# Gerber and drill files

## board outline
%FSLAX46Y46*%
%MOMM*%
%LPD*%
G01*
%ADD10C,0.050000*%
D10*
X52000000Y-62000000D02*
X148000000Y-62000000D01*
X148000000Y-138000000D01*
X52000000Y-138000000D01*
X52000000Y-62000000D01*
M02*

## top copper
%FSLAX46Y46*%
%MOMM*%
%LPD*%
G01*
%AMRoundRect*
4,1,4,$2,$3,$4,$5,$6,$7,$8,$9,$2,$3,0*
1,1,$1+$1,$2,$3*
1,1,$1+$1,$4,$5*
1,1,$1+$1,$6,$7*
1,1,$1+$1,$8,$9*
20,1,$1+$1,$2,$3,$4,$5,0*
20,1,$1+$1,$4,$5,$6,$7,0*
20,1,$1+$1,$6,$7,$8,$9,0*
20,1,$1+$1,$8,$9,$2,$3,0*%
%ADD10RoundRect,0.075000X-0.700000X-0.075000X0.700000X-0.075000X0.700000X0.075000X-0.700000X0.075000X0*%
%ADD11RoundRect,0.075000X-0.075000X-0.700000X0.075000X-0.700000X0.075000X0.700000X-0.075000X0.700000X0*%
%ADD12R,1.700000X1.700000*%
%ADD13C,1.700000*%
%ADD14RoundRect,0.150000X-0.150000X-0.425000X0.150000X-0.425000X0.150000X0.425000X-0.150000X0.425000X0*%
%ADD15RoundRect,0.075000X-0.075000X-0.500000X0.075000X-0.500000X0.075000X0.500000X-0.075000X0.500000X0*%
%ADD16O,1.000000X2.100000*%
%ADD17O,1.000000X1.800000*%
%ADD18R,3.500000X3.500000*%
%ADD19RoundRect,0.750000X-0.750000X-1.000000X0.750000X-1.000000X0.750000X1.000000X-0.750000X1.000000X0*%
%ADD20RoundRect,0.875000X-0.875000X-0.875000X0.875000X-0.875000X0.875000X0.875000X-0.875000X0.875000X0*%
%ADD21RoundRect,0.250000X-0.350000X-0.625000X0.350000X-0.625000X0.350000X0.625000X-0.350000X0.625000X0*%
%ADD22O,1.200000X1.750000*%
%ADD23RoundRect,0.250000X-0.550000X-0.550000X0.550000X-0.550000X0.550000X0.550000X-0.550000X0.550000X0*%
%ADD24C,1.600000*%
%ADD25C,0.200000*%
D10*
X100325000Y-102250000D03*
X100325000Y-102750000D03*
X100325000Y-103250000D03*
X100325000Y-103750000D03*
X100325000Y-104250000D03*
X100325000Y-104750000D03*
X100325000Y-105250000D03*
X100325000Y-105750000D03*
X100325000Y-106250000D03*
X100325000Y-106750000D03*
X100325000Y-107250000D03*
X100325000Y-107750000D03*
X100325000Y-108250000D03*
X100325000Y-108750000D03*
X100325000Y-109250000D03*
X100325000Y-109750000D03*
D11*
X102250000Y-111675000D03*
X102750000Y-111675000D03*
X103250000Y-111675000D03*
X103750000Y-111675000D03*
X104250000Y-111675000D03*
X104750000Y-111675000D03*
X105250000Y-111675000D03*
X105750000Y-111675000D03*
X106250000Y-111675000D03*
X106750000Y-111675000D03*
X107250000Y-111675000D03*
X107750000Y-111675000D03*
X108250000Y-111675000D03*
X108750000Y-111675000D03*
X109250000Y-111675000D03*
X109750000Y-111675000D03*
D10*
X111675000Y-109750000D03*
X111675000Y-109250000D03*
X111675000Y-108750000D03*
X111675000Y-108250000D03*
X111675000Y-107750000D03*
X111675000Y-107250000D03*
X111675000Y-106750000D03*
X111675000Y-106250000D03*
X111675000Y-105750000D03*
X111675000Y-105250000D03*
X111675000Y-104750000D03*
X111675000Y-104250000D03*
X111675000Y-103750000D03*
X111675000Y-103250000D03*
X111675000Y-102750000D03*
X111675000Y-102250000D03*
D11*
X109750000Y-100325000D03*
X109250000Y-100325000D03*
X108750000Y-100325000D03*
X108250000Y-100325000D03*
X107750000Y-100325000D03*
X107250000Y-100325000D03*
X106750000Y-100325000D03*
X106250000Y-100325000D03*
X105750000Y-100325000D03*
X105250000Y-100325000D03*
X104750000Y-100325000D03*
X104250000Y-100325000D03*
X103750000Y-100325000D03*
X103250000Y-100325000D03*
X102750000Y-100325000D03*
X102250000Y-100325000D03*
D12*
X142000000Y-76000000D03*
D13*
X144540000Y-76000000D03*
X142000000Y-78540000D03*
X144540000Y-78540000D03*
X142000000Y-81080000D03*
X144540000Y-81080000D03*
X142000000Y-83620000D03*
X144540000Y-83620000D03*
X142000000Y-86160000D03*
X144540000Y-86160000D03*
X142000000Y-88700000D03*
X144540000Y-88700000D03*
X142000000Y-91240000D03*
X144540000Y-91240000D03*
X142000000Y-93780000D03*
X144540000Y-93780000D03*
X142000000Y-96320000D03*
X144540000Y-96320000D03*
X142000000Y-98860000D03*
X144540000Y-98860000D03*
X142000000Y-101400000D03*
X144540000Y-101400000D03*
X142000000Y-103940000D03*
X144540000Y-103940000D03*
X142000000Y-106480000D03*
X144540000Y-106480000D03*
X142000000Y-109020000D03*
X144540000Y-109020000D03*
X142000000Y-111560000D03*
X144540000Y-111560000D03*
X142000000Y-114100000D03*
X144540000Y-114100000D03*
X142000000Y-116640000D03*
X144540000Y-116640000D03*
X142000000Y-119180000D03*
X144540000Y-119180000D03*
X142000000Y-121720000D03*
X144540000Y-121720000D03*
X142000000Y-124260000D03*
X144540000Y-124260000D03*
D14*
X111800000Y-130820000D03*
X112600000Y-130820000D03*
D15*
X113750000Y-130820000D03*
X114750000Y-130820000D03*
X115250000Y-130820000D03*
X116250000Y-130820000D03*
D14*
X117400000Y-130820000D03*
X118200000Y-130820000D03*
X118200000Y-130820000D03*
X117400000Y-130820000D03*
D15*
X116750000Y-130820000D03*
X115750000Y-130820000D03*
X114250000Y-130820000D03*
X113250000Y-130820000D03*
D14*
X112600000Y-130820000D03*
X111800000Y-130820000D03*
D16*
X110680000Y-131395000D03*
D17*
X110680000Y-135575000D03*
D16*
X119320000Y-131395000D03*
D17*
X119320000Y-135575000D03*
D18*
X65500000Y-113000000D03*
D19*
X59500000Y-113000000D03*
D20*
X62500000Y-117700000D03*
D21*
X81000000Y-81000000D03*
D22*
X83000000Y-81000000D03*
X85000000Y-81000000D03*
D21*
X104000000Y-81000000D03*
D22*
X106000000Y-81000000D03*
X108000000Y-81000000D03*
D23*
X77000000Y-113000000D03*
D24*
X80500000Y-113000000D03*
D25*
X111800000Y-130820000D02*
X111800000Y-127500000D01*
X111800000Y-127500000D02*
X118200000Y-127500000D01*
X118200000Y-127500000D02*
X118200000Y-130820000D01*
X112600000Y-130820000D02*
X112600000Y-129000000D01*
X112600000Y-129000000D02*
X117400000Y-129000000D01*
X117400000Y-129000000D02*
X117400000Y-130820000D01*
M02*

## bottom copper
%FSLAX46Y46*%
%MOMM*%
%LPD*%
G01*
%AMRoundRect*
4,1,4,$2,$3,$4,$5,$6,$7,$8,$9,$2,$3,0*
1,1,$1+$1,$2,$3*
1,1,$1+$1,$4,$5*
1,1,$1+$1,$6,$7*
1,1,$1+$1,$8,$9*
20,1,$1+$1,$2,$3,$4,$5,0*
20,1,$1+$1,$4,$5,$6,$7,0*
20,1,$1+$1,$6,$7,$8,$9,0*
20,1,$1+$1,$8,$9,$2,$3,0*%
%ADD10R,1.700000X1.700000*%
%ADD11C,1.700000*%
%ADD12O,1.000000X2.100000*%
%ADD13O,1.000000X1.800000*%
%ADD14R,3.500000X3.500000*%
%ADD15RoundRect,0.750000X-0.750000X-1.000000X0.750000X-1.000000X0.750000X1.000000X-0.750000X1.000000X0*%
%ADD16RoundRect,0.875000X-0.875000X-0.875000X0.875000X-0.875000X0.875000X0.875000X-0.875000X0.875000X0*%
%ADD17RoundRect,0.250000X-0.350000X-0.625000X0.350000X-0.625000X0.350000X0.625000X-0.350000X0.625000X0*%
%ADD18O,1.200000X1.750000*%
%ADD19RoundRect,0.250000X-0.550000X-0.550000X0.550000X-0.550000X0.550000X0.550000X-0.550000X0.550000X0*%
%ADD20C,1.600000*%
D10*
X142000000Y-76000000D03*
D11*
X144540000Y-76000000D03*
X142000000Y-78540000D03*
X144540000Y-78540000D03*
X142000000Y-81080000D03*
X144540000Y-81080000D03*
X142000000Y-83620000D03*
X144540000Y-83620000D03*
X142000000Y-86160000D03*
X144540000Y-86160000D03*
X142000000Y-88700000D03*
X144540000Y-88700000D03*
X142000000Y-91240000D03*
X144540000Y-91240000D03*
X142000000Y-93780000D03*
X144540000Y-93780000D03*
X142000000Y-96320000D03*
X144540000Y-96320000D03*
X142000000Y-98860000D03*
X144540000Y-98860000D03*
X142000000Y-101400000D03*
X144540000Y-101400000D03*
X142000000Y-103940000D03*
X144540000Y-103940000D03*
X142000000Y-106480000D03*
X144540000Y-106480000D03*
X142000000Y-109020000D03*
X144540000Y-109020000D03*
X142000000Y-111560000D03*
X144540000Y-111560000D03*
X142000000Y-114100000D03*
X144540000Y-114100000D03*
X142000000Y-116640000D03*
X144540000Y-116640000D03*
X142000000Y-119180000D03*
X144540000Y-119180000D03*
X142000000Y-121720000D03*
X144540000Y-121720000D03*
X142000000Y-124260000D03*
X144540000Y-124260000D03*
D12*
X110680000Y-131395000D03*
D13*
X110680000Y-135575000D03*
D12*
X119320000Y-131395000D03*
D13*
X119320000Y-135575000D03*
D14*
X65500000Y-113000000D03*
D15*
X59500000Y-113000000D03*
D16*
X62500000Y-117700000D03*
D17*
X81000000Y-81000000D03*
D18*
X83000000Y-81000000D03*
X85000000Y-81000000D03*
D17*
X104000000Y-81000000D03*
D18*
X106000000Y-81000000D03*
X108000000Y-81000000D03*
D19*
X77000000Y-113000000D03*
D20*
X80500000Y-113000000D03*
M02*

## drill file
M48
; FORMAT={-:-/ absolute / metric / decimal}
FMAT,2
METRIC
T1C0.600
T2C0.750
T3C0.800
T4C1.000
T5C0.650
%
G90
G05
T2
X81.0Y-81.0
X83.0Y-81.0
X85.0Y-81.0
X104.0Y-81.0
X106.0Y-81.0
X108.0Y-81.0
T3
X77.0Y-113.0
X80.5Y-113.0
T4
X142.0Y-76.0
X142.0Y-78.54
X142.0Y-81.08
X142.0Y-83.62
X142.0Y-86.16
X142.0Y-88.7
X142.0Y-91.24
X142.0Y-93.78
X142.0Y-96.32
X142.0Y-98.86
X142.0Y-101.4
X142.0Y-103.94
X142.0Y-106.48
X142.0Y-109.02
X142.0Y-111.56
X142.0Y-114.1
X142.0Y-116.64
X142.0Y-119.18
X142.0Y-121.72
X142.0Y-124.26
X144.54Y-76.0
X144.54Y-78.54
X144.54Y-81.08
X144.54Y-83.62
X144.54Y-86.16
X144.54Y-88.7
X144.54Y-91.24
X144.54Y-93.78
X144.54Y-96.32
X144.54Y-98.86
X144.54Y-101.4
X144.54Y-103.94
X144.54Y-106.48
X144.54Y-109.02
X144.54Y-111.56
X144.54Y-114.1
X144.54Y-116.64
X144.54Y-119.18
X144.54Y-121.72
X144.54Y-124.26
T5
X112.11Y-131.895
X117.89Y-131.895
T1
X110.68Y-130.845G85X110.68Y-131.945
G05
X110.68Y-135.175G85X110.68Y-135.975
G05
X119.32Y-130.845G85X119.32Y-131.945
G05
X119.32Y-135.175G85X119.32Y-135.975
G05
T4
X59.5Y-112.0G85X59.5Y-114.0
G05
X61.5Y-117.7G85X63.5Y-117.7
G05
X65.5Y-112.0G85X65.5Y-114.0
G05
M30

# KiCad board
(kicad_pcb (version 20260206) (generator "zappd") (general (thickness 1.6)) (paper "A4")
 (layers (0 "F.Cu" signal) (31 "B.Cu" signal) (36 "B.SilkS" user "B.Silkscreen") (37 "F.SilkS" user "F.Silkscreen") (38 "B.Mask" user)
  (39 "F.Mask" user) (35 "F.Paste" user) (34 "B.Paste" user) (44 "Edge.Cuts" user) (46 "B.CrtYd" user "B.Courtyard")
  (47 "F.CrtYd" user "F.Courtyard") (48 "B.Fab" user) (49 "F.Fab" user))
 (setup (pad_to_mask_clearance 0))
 (gr_rect (start 52.0 62.0) (end 148.0 138.0) (stroke (width 0.05) (type default)) (fill none) (layer "Edge.Cuts"))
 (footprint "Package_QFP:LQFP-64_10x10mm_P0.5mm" (layer "F.Cu") (at 106 106)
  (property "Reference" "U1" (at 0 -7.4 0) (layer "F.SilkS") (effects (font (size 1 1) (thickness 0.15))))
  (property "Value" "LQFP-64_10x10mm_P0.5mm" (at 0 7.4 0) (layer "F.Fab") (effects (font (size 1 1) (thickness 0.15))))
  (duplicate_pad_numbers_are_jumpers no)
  (pad "1" smd roundrect (at -5.675 -3.75) (size 1.55 0.3) (layers "F.Cu" "F.Mask" "F.Paste") (roundrect_rratio 0.25))
  (pad "2" smd roundrect (at -5.675 -3.25) (size 1.55 0.3) (layers "F.Cu" "F.Mask" "F.Paste") (roundrect_rratio 0.25))
  (pad "3" smd roundrect (at -5.675 -2.75) (size 1.55 0.3) (layers "F.Cu" "F.Mask" "F.Paste") (roundrect_rratio 0.25))
  (pad "4" smd roundrect (at -5.675 -2.25) (size 1.55 0.3) (layers "F.Cu" "F.Mask" "F.Paste") (roundrect_rratio 0.25))
  (pad "5" smd roundrect (at -5.675 -1.75) (size 1.55 0.3) (layers "F.Cu" "F.Mask" "F.Paste") (roundrect_rratio 0.25))
  (pad "6" smd roundrect (at -5.675 -1.25) (size 1.55 0.3) (layers "F.Cu" "F.Mask" "F.Paste") (roundrect_rratio 0.25))
  (pad "7" smd roundrect (at -5.675 -0.75) (size 1.55 0.3) (layers "F.Cu" "F.Mask" "F.Paste") (roundrect_rratio 0.25))
  (pad "8" smd roundrect (at -5.675 -0.25) (size 1.55 0.3) (layers "F.Cu" "F.Mask" "F.Paste") (roundrect_rratio 0.25))
  (pad "9" smd roundrect (at -5.675 0.25) (size 1.55 0.3) (layers "F.Cu" "F.Mask" "F.Paste") (roundrect_rratio 0.25))
  (pad "10" smd roundrect (at -5.675 0.75) (size 1.55 0.3) (layers "F.Cu" "F.Mask" "F.Paste") (roundrect_rratio 0.25))
  (pad "11" smd roundrect (at -5.675 1.25) (size 1.55 0.3) (layers "F.Cu" "F.Mask" "F.Paste") (roundrect_rratio 0.25))
  (pad "12" smd roundrect (at -5.675 1.75) (size 1.55 0.3) (layers "F.Cu" "F.Mask" "F.Paste") (roundrect_rratio 0.25))
  (pad "13" smd roundrect (at -5.675 2.25) (size 1.55 0.3) (layers "F.Cu" "F.Mask" "F.Paste") (roundrect_rratio 0.25))
  (pad "14" smd roundrect (at -5.675 2.75) (size 1.55 0.3) (layers "F.Cu" "F.Mask" "F.Paste") (roundrect_rratio 0.25))
  (pad "15" smd roundrect (at -5.675 3.25) (size 1.55 0.3) (layers "F.Cu" "F.Mask" "F.Paste") (roundrect_rratio 0.25))
  (pad "16" smd roundrect (at -5.675 3.75) (size 1.55 0.3) (layers "F.Cu" "F.Mask" "F.Paste") (roundrect_rratio 0.25))
  (pad "17" smd roundrect (at -3.75 5.675) (size 0.3 1.55) (layers "F.Cu" "F.Mask" "F.Paste") (roundrect_rratio 0.25))
  (pad "18" smd roundrect (at -3.25 5.675) (size 0.3 1.55) (layers "F.Cu" "F.Mask" "F.Paste") (roundrect_rratio 0.25))
  (pad "19" smd roundrect (at -2.75 5.675) (size 0.3 1.55) (layers "F.Cu" "F.Mask" "F.Paste") (roundrect_rratio 0.25))
  (pad "20" smd roundrect (at -2.25 5.675) (size 0.3 1.55) (layers "F.Cu" "F.Mask" "F.Paste") (roundrect_rratio 0.25))
  (pad "21" smd roundrect (at -1.75 5.675) (size 0.3 1.55) (layers "F.Cu" "F.Mask" "F.Paste") (roundrect_rratio 0.25))
  (pad "22" smd roundrect (at -1.25 5.675) (size 0.3 1.55) (layers "F.Cu" "F.Mask" "F.Paste") (roundrect_rratio 0.25))
  (pad "23" smd roundrect (at -0.75 5.675) (size 0.3 1.55) (layers "F.Cu" "F.Mask" "F.Paste") (roundrect_rratio 0.25))
  (pad "24" smd roundrect (at -0.25 5.675) (size 0.3 1.55) (layers "F.Cu" "F.Mask" "F.Paste") (roundrect_rratio 0.25))
  (pad "25" smd roundrect (at 0.25 5.675) (size 0.3 1.55) (layers "F.Cu" "F.Mask" "F.Paste") (roundrect_rratio 0.25))
  (pad "26" smd roundrect (at 0.75 5.675) (size 0.3 1.55) (layers "F.Cu" "F.Mask" "F.Paste") (roundrect_rratio 0.25))
  (pad "27" smd roundrect (at 1.25 5.675) (size 0.3 1.55) (layers "F.Cu" "F.Mask" "F.Paste") (roundrect_rratio 0.25))
  (pad "28" smd roundrect (at 1.75 5.675) (size 0.3 1.55) (layers "F.Cu" "F.Mask" "F.Paste") (roundrect_rratio 0.25))
  (pad "29" smd roundrect (at 2.25 5.675) (size 0.3 1.55) (layers "F.Cu" "F.Mask" "F.Paste") (roundrect_rratio 0.25))
  (pad "30" smd roundrect (at 2.75 5.675) (size 0.3 1.55) (layers "F.Cu" "F.Mask" "F.Paste") (roundrect_rratio 0.25))
  (pad "31" smd roundrect (at 3.25 5.675) (size 0.3 1.55) (layers "F.Cu" "F.Mask" "F.Paste") (roundrect_rratio 0.25))
  (pad "32" smd roundrect (at 3.75 5.675) (size 0.3 1.55) (layers "F.Cu" "F.Mask" "F.Paste") (roundrect_rratio 0.25))
  (pad "33" smd roundrect (at 5.675 3.75) (size 1.55 0.3) (layers "F.Cu" "F.Mask" "F.Paste") (roundrect_rratio 0.25))
  (pad "34" smd roundrect (at 5.675 3.25) (size 1.55 0.3) (layers "F.Cu" "F.Mask" "F.Paste") (roundrect_rratio 0.25))
  (pad "35" smd roundrect (at 5.675 2.75) (size 1.55 0.3) (layers "F.Cu" "F.Mask" "F.Paste") (roundrect_rratio 0.25))
  (pad "36" smd roundrect (at 5.675 2.25) (size 1.55 0.3) (layers "F.Cu" "F.Mask" "F.Paste") (roundrect_rratio 0.25))
  (pad "37" smd roundrect (at 5.675 1.75) (size 1.55 0.3) (layers "F.Cu" "F.Mask" "F.Paste") (roundrect_rratio 0.25))
  (pad "38" smd roundrect (at 5.675 1.25) (size 1.55 0.3) (layers "F.Cu" "F.Mask" "F.Paste") (roundrect_rratio 0.25))
  (pad "39" smd roundrect (at 5.675 0.75) (size 1.55 0.3) (layers "F.Cu" "F.Mask" "F.Paste") (roundrect_rratio 0.25))
  (pad "40" smd roundrect (at 5.675 0.25) (size 1.55 0.3) (layers "F.Cu" "F.Mask" "F.Paste") (roundrect_rratio 0.25))
  (pad "41" smd roundrect (at 5.675 -0.25) (size 1.55 0.3) (layers "F.Cu" "F.Mask" "F.Paste") (roundrect_rratio 0.25))
  (pad "42" smd roundrect (at 5.675 -0.75) (size 1.55 0.3) (layers "F.Cu" "F.Mask" "F.Paste") (roundrect_rratio 0.25))
  (pad "43" smd roundrect (at 5.675 -1.25) (size 1.55 0.3) (layers "F.Cu" "F.Mask" "F.Paste") (roundrect_rratio 0.25))
  (pad "44" smd roundrect (at 5.675 -1.75) (size 1.55 0.3) (layers "F.Cu" "F.Mask" "F.Paste") (roundrect_rratio 0.25))
  (pad "45" smd roundrect (at 5.675 -2.25) (size 1.55 0.3) (layers "F.Cu" "F.Mask" "F.Paste") (roundrect_rratio 0.25))
  (pad "46" smd roundrect (at 5.675 -2.75) (size 1.55 0.3) (layers "F.Cu" "F.Mask" "F.Paste") (roundrect_rratio 0.25))
  (pad "47" smd roundrect (at 5.675 -3.25) (size 1.55 0.3) (layers "F.Cu" "F.Mask" "F.Paste") (roundrect_rratio 0.25))
  (pad "48" smd roundrect (at 5.675 -3.75) (size 1.55 0.3) (layers "F.Cu" "F.Mask" "F.Paste") (roundrect_rratio 0.25))
  (pad "49" smd roundrect (at 3.75 -5.675) (size 0.3 1.55) (layers "F.Cu" "F.Mask" "F.Paste") (roundrect_rratio 0.25))
  (pad "50" smd roundrect (at 3.25 -5.675) (size 0.3 1.55) (layers "F.Cu" "F.Mask" "F.Paste") (roundrect_rratio 0.25))
  (pad "51" smd roundrect (at 2.75 -5.675) (size 0.3 1.55) (layers "F.Cu" "F.Mask" "F.Paste") (roundrect_rratio 0.25))
  (pad "52" smd roundrect (at 2.25 -5.675) (size 0.3 1.55) (layers "F.Cu" "F.Mask" "F.Paste") (roundrect_rratio 0.25))
  (pad "53" smd roundrect (at 1.75 -5.675) (size 0.3 1.55) (layers "F.Cu" "F.Mask" "F.Paste") (roundrect_rratio 0.25))
  (pad "54" smd roundrect (at 1.25 -5.675) (size 0.3 1.55) (layers "F.Cu" "F.Mask" "F.Paste") (roundrect_rratio 0.25))
  (pad "55" smd roundrect (at 0.75 -5.675) (size 0.3 1.55) (layers "F.Cu" "F.Mask" "F.Paste") (roundrect_rratio 0.25))
  (pad "56" smd roundrect (at 0.25 -5.675) (size 0.3 1.55) (layers "F.Cu" "F.Mask" "F.Paste") (roundrect_rratio 0.25))
  (pad "57" smd roundrect (at -0.25 -5.675) (size 0.3 1.55) (layers "F.Cu" "F.Mask" "F.Paste") (roundrect_rratio 0.25))
  (pad "58" smd roundrect (at -0.75 -5.675) (size 0.3 1.55) (layers "F.Cu" "F.Mask" "F.Paste") (roundrect_rratio 0.25))
  (pad "59" smd roundrect (at -1.25 -5.675) (size 0.3 1.55) (layers "F.Cu" "F.Mask" "F.Paste") (roundrect_rratio 0.25))
  (pad "60" smd roundrect (at -1.75 -5.675) (size 0.3 1.55) (layers "F.Cu" "F.Mask" "F.Paste") (roundrect_rratio 0.25))
  (pad "61" smd roundrect (at -2.25 -5.675) (size 0.3 1.55) (layers "F.Cu" "F.Mask" "F.Paste") (roundrect_rratio 0.25))
  (pad "62" smd roundrect (at -2.75 -5.675) (size 0.3 1.55) (layers "F.Cu" "F.Mask" "F.Paste") (roundrect_rratio 0.25))
  (pad "63" smd roundrect (at -3.25 -5.675) (size 0.3 1.55) (layers "F.Cu" "F.Mask" "F.Paste") (roundrect_rratio 0.25))
  (pad "64" smd roundrect (at -3.75 -5.675) (size 0.3 1.55) (layers "F.Cu" "F.Mask" "F.Paste") (roundrect_rratio 0.25)))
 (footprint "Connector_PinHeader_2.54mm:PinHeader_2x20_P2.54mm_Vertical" (layer "F.Cu") (at 142 76)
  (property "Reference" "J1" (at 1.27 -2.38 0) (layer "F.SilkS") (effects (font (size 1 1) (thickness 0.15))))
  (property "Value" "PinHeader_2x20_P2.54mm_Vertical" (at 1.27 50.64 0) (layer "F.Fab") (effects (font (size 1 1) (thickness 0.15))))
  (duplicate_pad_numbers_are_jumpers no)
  (pad "1" thru_hole rect (at 0 0) (size 1.7 1.7) (drill 1) (layers "*.Cu" "*.Mask") (remove_unused_layers no))
  (pad "2" thru_hole circle (at 2.54 0) (size 1.7 1.7) (drill 1) (layers "*.Cu" "*.Mask") (remove_unused_layers no))
  (pad "3" thru_hole circle (at 0 2.54) (size 1.7 1.7) (drill 1) (layers "*.Cu" "*.Mask") (remove_unused_layers no))
  (pad "4" thru_hole circle (at 2.54 2.54) (size 1.7 1.7) (drill 1) (layers "*.Cu" "*.Mask") (remove_unused_layers no))
  (pad "5" thru_hole circle (at 0 5.08) (size 1.7 1.7) (drill 1) (layers "*.Cu" "*.Mask") (remove_unused_layers no))
  (pad "6" thru_hole circle (at 2.54 5.08) (size 1.7 1.7) (drill 1) (layers "*.Cu" "*.Mask") (remove_unused_layers no))
  (pad "7" thru_hole circle (at 0 7.62) (size 1.7 1.7) (drill 1) (layers "*.Cu" "*.Mask") (remove_unused_layers no))
  (pad "8" thru_hole circle (at 2.54 7.62) (size 1.7 1.7) (drill 1) (layers "*.Cu" "*.Mask") (remove_unused_layers no))
  (pad "9" thru_hole circle (at 0 10.16) (size 1.7 1.7) (drill 1) (layers "*.Cu" "*.Mask") (remove_unused_layers no))
  (pad "10" thru_hole circle (at 2.54 10.16) (size 1.7 1.7) (drill 1) (layers "*.Cu" "*.Mask") (remove_unused_layers no))
  (pad "11" thru_hole circle (at 0 12.7) (size 1.7 1.7) (drill 1) (layers "*.Cu" "*.Mask") (remove_unused_layers no))
  (pad "12" thru_hole circle (at 2.54 12.7) (size 1.7 1.7) (drill 1) (layers "*.Cu" "*.Mask") (remove_unused_layers no))
  (pad "13" thru_hole circle (at 0 15.24) (size 1.7 1.7) (drill 1) (layers "*.Cu" "*.Mask") (remove_unused_layers no))
  (pad "14" thru_hole circle (at 2.54 15.24) (size 1.7 1.7) (drill 1) (layers "*.Cu" "*.Mask") (remove_unused_layers no))
  (pad "15" thru_hole circle (at 0 17.78) (size 1.7 1.7) (drill 1) (layers "*.Cu" "*.Mask") (remove_unused_layers no))
  (pad "16" thru_hole circle (at 2.54 17.78) (size 1.7 1.7) (drill 1) (layers "*.Cu" "*.Mask") (remove_unused_layers no))
  (pad "17" thru_hole circle (at 0 20.32) (size 1.7 1.7) (drill 1) (layers "*.Cu" "*.Mask") (remove_unused_layers no))
  (pad "18" thru_hole circle (at 2.54 20.32) (size 1.7 1.7) (drill 1) (layers "*.Cu" "*.Mask") (remove_unused_layers no))
  (pad "19" thru_hole circle (at 0 22.86) (size 1.7 1.7) (drill 1) (layers "*.Cu" "*.Mask") (remove_unused_layers no))
  (pad "20" thru_hole circle (at 2.54 22.86) (size 1.7 1.7) (drill 1) (layers "*.Cu" "*.Mask") (remove_unused_layers no))
  (pad "21" thru_hole circle (at 0 25.4) (size 1.7 1.7) (drill 1) (layers "*.Cu" "*.Mask") (remove_unused_layers no))
  (pad "22" thru_hole circle (at 2.54 25.4) (size 1.7 1.7) (drill 1) (layers "*.Cu" "*.Mask") (remove_unused_layers no))
  (pad "23" thru_hole circle (at 0 27.94) (size 1.7 1.7) (drill 1) (layers "*.Cu" "*.Mask") (remove_unused_layers no))
  (pad "24" thru_hole circle (at 2.54 27.94) (size 1.7 1.7) (drill 1) (layers "*.Cu" "*.Mask") (remove_unused_layers no))
  (pad "25" thru_hole circle (at 0 30.48) (size 1.7 1.7) (drill 1) (layers "*.Cu" "*.Mask") (remove_unused_layers no))
  (pad "26" thru_hole circle (at 2.54 30.48) (size 1.7 1.7) (drill 1) (layers "*.Cu" "*.Mask") (remove_unused_layers no))
  (pad "27" thru_hole circle (at 0 33.02) (size 1.7 1.7) (drill 1) (layers "*.Cu" "*.Mask") (remove_unused_layers no))
  (pad "28" thru_hole circle (at 2.54 33.02) (size 1.7 1.7) (drill 1) (layers "*.Cu" "*.Mask") (remove_unused_layers no))
  (pad "29" thru_hole circle (at 0 35.56) (size 1.7 1.7) (drill 1) (layers "*.Cu" "*.Mask") (remove_unused_layers no))
  (pad "30" thru_hole circle (at 2.54 35.56) (size 1.7 1.7) (drill 1) (layers "*.Cu" "*.Mask") (remove_unused_layers no))
  (pad "31" thru_hole circle (at 0 38.1) (size 1.7 1.7) (drill 1) (layers "*.Cu" "*.Mask") (remove_unused_layers no))
  (pad "32" thru_hole circle (at 2.54 38.1) (size 1.7 1.7) (drill 1) (layers "*.Cu" "*.Mask") (remove_unused_layers no))
  (pad "33" thru_hole circle (at 0 40.64) (size 1.7 1.7) (drill 1) (layers "*.Cu" "*.Mask") (remove_unused_layers no))
  (pad "34" thru_hole circle (at 2.54 40.64) (size 1.7 1.7) (drill 1) (layers "*.Cu" "*.Mask") (remove_unused_layers no))
  (pad "35" thru_hole circle (at 0 43.18) (size 1.7 1.7) (drill 1) (layers "*.Cu" "*.Mask") (remove_unused_layers no))
  (pad "36" thru_hole circle (at 2.54 43.18) (size 1.7 1.7) (drill 1) (layers "*.Cu" "*.Mask") (remove_unused_layers no))
  (pad "37" thru_hole circle (at 0 45.72) (size 1.7 1.7) (drill 1) (layers "*.Cu" "*.Mask") (remove_unused_layers no))
  (pad "38" thru_hole circle (at 2.54 45.72) (size 1.7 1.7) (drill 1) (layers "*.Cu" "*.Mask") (remove_unused_layers no))
  (pad "39" thru_hole circle (at 0 48.26) (size 1.7 1.7) (drill 1) (layers "*.Cu" "*.Mask") (remove_unused_layers no))
  (pad "40" thru_hole circle (at 2.54 48.26) (size 1.7 1.7) (drill 1) (layers "*.Cu" "*.Mask") (remove_unused_layers no)))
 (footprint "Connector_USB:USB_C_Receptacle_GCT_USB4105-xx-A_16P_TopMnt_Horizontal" (layer "F.Cu") (at 115 134.5)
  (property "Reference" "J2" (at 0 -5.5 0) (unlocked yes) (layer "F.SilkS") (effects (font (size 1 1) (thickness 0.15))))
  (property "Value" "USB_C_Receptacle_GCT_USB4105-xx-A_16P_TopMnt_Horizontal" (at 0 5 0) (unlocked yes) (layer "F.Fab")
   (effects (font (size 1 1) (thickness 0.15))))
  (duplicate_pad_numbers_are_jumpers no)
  (pad "" np_thru_hole circle (at -2.89 -2.605) (size 0.65 0.65) (drill 0.65) (layers "*.Cu" "*.Mask"))
  (pad "" np_thru_hole circle (at 2.89 -2.605) (size 0.65 0.65) (drill 0.65) (layers "*.Cu" "*.Mask"))
  (pad "A1" smd roundrect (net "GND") (at -3.2 -3.68) (size 0.6 1.15) (layers "F.Cu" "F.Mask" "F.Paste") (roundrect_rratio 0.25))
  (pad "A4" smd roundrect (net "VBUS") (at -2.4 -3.68) (size 0.6 1.15) (layers "F.Cu" "F.Mask" "F.Paste") (roundrect_rratio 0.25))
  (pad "A5" smd roundrect (at -1.25 -3.68) (size 0.3 1.15) (layers "F.Cu" "F.Mask" "F.Paste") (roundrect_rratio 0.25))
  (pad "A6" smd roundrect (at -0.25 -3.68) (size 0.3 1.15) (layers "F.Cu" "F.Mask" "F.Paste") (roundrect_rratio 0.25))
  (pad "A7" smd roundrect (at 0.25 -3.68) (size 0.3 1.15) (layers "F.Cu" "F.Mask" "F.Paste") (roundrect_rratio 0.25))
  (pad "A8" smd roundrect (at 1.25 -3.68) (size 0.3 1.15) (layers "F.Cu" "F.Mask" "F.Paste") (roundrect_rratio 0.25))
  (pad "A9" smd roundrect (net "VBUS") (at 2.4 -3.68) (size 0.6 1.15) (layers "F.Cu" "F.Mask" "F.Paste") (roundrect_rratio 0.25))
  (pad "A12" smd roundrect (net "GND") (at 3.2 -3.68) (size 0.6 1.15) (layers "F.Cu" "F.Mask" "F.Paste") (roundrect_rratio 0.25))
  (pad "B1" smd roundrect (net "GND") (at 3.2 -3.68) (size 0.6 1.15) (layers "F.Cu" "F.Mask" "F.Paste") (roundrect_rratio 0.25))
  (pad "B4" smd roundrect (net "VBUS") (at 2.4 -3.68) (size 0.6 1.15) (layers "F.Cu" "F.Mask" "F.Paste") (roundrect_rratio 0.25))
  (pad "B5" smd roundrect (at 1.75 -3.68) (size 0.3 1.15) (layers "F.Cu" "F.Mask" "F.Paste") (roundrect_rratio 0.25))
  (pad "B6" smd roundrect (at 0.75 -3.68) (size 0.3 1.15) (layers "F.Cu" "F.Mask" "F.Paste") (roundrect_rratio 0.25))
  (pad "B7" smd roundrect (at -0.75 -3.68) (size 0.3 1.15) (layers "F.Cu" "F.Mask" "F.Paste") (roundrect_rratio 0.25))
  (pad "B8" smd roundrect (at -1.75 -3.68) (size 0.3 1.15) (layers "F.Cu" "F.Mask" "F.Paste") (roundrect_rratio 0.25))
  (pad "B9" smd roundrect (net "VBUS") (at -2.4 -3.68) (size 0.6 1.15) (layers "F.Cu" "F.Mask" "F.Paste") (roundrect_rratio 0.25))
  (pad "B12" smd roundrect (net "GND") (at -3.2 -3.68) (size 0.6 1.15) (layers "F.Cu" "F.Mask" "F.Paste") (roundrect_rratio 0.25))
  (pad "SH" thru_hole oval (at -4.32 -3.105) (size 1 2.1) (drill oval 0.6 1.7) (layers "*.Cu" "*.Mask" "F.Paste") (remove_unused_layers no))
  (pad "SH" thru_hole oval (at -4.32 1.075) (size 1 1.8) (drill oval 0.6 1.4) (layers "*.Cu" "*.Mask" "F.Paste") (remove_unused_layers no))
  (pad "SH" thru_hole oval (at 4.32 -3.105) (size 1 2.1) (drill oval 0.6 1.7) (layers "*.Cu" "*.Mask" "F.Paste") (remove_unused_layers no))
  (pad "SH" thru_hole oval (at 4.32 1.075) (size 1 1.8) (drill oval 0.6 1.4) (layers "*.Cu" "*.Mask" "F.Paste") (remove_unused_layers no)))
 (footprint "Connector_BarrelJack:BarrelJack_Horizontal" (layer "F.Cu") (at 65.5 113)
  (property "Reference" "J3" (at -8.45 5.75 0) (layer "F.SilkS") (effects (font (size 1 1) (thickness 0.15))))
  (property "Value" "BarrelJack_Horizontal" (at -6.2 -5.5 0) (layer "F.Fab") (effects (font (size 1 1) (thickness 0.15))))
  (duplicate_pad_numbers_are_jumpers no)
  (pad "1" thru_hole rect (at 0 0) (size 3.5 3.5) (drill oval 1 3) (layers "*.Cu" "*.Mask") (remove_unused_layers no))
  (pad "2" thru_hole roundrect (at -6 0) (size 3 3.5) (drill oval 1 3) (layers "*.Cu" "*.Mask") (remove_unused_layers no)
   (roundrect_rratio 0.25))
  (pad "3" thru_hole roundrect (at -3 4.7) (size 3.5 3.5) (drill oval 3 1) (layers "*.Cu" "*.Mask") (remove_unused_layers no)
   (roundrect_rratio 0.25)))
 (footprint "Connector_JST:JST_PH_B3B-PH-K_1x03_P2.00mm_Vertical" (layer "F.Cu") (at 81 81)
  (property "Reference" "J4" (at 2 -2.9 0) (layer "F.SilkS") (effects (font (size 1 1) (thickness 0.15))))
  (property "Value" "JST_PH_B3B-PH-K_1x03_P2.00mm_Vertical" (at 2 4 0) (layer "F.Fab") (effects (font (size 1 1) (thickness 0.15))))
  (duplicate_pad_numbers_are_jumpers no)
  (pad "1" thru_hole roundrect (at 0 0) (size 1.2 1.75) (drill 0.75) (layers "*.Cu" "*.Mask") (remove_unused_layers no)
   (roundrect_rratio 0.208333))
  (pad "2" thru_hole oval (at 2 0) (size 1.2 1.75) (drill 0.75) (layers "*.Cu" "*.Mask") (remove_unused_layers no))
  (pad "3" thru_hole oval (at 4 0) (size 1.2 1.75) (drill 0.75) (layers "*.Cu" "*.Mask") (remove_unused_layers no)))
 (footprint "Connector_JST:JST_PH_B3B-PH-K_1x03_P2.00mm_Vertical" (layer "F.Cu") (at 104 81)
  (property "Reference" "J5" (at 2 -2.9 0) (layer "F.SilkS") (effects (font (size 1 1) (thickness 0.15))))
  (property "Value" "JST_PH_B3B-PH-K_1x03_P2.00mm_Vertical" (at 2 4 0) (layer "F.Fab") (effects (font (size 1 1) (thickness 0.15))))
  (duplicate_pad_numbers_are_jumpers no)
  (pad "1" thru_hole roundrect (at 0 0) (size 1.2 1.75) (drill 0.75) (layers "*.Cu" "*.Mask") (remove_unused_layers no)
   (roundrect_rratio 0.208333))
  (pad "2" thru_hole oval (at 2 0) (size 1.2 1.75) (drill 0.75) (layers "*.Cu" "*.Mask") (remove_unused_layers no))
  (pad "3" thru_hole oval (at 4 0) (size 1.2 1.75) (drill 0.75) (layers "*.Cu" "*.Mask") (remove_unused_layers no)))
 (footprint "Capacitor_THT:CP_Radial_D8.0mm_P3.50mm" (layer "F.Cu") (at 77 113)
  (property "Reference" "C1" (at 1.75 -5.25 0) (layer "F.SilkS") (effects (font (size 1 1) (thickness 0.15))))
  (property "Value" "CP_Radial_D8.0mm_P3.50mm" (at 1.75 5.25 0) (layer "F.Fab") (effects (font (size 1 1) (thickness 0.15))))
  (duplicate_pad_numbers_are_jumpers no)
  (pad "1" thru_hole roundrect (at 0 0) (size 1.6 1.6) (drill 0.8) (layers "*.Cu" "*.Mask") (remove_unused_layers no)
   (roundrect_rratio 0.15625))
  (pad "2" thru_hole circle (at 3.5 0) (size 1.6 1.6) (drill 0.8) (layers "*.Cu" "*.Mask") (remove_unused_layers no)))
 (segment (start 111.8000 130.8200) (end 111.8000 127.5000) (width 0.2) (layer "F.Cu") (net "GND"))
 (segment (start 111.8000 127.5000) (end 118.2000 127.5000) (width 0.2) (layer "F.Cu") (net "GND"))
 (segment (start 118.2000 127.5000) (end 118.2000 130.8200) (width 0.2) (layer "F.Cu") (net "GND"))
 (segment (start 112.6000 130.8200) (end 112.6000 129.0000) (width 0.2) (layer "F.Cu") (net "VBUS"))
 (segment (start 112.6000 129.0000) (end 117.4000 129.0000) (width 0.2) (layer "F.Cu") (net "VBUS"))
 (segment (start 117.4000 129.0000) (end 117.4000 130.8200) (width 0.2) (layer "F.Cu") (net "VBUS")))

